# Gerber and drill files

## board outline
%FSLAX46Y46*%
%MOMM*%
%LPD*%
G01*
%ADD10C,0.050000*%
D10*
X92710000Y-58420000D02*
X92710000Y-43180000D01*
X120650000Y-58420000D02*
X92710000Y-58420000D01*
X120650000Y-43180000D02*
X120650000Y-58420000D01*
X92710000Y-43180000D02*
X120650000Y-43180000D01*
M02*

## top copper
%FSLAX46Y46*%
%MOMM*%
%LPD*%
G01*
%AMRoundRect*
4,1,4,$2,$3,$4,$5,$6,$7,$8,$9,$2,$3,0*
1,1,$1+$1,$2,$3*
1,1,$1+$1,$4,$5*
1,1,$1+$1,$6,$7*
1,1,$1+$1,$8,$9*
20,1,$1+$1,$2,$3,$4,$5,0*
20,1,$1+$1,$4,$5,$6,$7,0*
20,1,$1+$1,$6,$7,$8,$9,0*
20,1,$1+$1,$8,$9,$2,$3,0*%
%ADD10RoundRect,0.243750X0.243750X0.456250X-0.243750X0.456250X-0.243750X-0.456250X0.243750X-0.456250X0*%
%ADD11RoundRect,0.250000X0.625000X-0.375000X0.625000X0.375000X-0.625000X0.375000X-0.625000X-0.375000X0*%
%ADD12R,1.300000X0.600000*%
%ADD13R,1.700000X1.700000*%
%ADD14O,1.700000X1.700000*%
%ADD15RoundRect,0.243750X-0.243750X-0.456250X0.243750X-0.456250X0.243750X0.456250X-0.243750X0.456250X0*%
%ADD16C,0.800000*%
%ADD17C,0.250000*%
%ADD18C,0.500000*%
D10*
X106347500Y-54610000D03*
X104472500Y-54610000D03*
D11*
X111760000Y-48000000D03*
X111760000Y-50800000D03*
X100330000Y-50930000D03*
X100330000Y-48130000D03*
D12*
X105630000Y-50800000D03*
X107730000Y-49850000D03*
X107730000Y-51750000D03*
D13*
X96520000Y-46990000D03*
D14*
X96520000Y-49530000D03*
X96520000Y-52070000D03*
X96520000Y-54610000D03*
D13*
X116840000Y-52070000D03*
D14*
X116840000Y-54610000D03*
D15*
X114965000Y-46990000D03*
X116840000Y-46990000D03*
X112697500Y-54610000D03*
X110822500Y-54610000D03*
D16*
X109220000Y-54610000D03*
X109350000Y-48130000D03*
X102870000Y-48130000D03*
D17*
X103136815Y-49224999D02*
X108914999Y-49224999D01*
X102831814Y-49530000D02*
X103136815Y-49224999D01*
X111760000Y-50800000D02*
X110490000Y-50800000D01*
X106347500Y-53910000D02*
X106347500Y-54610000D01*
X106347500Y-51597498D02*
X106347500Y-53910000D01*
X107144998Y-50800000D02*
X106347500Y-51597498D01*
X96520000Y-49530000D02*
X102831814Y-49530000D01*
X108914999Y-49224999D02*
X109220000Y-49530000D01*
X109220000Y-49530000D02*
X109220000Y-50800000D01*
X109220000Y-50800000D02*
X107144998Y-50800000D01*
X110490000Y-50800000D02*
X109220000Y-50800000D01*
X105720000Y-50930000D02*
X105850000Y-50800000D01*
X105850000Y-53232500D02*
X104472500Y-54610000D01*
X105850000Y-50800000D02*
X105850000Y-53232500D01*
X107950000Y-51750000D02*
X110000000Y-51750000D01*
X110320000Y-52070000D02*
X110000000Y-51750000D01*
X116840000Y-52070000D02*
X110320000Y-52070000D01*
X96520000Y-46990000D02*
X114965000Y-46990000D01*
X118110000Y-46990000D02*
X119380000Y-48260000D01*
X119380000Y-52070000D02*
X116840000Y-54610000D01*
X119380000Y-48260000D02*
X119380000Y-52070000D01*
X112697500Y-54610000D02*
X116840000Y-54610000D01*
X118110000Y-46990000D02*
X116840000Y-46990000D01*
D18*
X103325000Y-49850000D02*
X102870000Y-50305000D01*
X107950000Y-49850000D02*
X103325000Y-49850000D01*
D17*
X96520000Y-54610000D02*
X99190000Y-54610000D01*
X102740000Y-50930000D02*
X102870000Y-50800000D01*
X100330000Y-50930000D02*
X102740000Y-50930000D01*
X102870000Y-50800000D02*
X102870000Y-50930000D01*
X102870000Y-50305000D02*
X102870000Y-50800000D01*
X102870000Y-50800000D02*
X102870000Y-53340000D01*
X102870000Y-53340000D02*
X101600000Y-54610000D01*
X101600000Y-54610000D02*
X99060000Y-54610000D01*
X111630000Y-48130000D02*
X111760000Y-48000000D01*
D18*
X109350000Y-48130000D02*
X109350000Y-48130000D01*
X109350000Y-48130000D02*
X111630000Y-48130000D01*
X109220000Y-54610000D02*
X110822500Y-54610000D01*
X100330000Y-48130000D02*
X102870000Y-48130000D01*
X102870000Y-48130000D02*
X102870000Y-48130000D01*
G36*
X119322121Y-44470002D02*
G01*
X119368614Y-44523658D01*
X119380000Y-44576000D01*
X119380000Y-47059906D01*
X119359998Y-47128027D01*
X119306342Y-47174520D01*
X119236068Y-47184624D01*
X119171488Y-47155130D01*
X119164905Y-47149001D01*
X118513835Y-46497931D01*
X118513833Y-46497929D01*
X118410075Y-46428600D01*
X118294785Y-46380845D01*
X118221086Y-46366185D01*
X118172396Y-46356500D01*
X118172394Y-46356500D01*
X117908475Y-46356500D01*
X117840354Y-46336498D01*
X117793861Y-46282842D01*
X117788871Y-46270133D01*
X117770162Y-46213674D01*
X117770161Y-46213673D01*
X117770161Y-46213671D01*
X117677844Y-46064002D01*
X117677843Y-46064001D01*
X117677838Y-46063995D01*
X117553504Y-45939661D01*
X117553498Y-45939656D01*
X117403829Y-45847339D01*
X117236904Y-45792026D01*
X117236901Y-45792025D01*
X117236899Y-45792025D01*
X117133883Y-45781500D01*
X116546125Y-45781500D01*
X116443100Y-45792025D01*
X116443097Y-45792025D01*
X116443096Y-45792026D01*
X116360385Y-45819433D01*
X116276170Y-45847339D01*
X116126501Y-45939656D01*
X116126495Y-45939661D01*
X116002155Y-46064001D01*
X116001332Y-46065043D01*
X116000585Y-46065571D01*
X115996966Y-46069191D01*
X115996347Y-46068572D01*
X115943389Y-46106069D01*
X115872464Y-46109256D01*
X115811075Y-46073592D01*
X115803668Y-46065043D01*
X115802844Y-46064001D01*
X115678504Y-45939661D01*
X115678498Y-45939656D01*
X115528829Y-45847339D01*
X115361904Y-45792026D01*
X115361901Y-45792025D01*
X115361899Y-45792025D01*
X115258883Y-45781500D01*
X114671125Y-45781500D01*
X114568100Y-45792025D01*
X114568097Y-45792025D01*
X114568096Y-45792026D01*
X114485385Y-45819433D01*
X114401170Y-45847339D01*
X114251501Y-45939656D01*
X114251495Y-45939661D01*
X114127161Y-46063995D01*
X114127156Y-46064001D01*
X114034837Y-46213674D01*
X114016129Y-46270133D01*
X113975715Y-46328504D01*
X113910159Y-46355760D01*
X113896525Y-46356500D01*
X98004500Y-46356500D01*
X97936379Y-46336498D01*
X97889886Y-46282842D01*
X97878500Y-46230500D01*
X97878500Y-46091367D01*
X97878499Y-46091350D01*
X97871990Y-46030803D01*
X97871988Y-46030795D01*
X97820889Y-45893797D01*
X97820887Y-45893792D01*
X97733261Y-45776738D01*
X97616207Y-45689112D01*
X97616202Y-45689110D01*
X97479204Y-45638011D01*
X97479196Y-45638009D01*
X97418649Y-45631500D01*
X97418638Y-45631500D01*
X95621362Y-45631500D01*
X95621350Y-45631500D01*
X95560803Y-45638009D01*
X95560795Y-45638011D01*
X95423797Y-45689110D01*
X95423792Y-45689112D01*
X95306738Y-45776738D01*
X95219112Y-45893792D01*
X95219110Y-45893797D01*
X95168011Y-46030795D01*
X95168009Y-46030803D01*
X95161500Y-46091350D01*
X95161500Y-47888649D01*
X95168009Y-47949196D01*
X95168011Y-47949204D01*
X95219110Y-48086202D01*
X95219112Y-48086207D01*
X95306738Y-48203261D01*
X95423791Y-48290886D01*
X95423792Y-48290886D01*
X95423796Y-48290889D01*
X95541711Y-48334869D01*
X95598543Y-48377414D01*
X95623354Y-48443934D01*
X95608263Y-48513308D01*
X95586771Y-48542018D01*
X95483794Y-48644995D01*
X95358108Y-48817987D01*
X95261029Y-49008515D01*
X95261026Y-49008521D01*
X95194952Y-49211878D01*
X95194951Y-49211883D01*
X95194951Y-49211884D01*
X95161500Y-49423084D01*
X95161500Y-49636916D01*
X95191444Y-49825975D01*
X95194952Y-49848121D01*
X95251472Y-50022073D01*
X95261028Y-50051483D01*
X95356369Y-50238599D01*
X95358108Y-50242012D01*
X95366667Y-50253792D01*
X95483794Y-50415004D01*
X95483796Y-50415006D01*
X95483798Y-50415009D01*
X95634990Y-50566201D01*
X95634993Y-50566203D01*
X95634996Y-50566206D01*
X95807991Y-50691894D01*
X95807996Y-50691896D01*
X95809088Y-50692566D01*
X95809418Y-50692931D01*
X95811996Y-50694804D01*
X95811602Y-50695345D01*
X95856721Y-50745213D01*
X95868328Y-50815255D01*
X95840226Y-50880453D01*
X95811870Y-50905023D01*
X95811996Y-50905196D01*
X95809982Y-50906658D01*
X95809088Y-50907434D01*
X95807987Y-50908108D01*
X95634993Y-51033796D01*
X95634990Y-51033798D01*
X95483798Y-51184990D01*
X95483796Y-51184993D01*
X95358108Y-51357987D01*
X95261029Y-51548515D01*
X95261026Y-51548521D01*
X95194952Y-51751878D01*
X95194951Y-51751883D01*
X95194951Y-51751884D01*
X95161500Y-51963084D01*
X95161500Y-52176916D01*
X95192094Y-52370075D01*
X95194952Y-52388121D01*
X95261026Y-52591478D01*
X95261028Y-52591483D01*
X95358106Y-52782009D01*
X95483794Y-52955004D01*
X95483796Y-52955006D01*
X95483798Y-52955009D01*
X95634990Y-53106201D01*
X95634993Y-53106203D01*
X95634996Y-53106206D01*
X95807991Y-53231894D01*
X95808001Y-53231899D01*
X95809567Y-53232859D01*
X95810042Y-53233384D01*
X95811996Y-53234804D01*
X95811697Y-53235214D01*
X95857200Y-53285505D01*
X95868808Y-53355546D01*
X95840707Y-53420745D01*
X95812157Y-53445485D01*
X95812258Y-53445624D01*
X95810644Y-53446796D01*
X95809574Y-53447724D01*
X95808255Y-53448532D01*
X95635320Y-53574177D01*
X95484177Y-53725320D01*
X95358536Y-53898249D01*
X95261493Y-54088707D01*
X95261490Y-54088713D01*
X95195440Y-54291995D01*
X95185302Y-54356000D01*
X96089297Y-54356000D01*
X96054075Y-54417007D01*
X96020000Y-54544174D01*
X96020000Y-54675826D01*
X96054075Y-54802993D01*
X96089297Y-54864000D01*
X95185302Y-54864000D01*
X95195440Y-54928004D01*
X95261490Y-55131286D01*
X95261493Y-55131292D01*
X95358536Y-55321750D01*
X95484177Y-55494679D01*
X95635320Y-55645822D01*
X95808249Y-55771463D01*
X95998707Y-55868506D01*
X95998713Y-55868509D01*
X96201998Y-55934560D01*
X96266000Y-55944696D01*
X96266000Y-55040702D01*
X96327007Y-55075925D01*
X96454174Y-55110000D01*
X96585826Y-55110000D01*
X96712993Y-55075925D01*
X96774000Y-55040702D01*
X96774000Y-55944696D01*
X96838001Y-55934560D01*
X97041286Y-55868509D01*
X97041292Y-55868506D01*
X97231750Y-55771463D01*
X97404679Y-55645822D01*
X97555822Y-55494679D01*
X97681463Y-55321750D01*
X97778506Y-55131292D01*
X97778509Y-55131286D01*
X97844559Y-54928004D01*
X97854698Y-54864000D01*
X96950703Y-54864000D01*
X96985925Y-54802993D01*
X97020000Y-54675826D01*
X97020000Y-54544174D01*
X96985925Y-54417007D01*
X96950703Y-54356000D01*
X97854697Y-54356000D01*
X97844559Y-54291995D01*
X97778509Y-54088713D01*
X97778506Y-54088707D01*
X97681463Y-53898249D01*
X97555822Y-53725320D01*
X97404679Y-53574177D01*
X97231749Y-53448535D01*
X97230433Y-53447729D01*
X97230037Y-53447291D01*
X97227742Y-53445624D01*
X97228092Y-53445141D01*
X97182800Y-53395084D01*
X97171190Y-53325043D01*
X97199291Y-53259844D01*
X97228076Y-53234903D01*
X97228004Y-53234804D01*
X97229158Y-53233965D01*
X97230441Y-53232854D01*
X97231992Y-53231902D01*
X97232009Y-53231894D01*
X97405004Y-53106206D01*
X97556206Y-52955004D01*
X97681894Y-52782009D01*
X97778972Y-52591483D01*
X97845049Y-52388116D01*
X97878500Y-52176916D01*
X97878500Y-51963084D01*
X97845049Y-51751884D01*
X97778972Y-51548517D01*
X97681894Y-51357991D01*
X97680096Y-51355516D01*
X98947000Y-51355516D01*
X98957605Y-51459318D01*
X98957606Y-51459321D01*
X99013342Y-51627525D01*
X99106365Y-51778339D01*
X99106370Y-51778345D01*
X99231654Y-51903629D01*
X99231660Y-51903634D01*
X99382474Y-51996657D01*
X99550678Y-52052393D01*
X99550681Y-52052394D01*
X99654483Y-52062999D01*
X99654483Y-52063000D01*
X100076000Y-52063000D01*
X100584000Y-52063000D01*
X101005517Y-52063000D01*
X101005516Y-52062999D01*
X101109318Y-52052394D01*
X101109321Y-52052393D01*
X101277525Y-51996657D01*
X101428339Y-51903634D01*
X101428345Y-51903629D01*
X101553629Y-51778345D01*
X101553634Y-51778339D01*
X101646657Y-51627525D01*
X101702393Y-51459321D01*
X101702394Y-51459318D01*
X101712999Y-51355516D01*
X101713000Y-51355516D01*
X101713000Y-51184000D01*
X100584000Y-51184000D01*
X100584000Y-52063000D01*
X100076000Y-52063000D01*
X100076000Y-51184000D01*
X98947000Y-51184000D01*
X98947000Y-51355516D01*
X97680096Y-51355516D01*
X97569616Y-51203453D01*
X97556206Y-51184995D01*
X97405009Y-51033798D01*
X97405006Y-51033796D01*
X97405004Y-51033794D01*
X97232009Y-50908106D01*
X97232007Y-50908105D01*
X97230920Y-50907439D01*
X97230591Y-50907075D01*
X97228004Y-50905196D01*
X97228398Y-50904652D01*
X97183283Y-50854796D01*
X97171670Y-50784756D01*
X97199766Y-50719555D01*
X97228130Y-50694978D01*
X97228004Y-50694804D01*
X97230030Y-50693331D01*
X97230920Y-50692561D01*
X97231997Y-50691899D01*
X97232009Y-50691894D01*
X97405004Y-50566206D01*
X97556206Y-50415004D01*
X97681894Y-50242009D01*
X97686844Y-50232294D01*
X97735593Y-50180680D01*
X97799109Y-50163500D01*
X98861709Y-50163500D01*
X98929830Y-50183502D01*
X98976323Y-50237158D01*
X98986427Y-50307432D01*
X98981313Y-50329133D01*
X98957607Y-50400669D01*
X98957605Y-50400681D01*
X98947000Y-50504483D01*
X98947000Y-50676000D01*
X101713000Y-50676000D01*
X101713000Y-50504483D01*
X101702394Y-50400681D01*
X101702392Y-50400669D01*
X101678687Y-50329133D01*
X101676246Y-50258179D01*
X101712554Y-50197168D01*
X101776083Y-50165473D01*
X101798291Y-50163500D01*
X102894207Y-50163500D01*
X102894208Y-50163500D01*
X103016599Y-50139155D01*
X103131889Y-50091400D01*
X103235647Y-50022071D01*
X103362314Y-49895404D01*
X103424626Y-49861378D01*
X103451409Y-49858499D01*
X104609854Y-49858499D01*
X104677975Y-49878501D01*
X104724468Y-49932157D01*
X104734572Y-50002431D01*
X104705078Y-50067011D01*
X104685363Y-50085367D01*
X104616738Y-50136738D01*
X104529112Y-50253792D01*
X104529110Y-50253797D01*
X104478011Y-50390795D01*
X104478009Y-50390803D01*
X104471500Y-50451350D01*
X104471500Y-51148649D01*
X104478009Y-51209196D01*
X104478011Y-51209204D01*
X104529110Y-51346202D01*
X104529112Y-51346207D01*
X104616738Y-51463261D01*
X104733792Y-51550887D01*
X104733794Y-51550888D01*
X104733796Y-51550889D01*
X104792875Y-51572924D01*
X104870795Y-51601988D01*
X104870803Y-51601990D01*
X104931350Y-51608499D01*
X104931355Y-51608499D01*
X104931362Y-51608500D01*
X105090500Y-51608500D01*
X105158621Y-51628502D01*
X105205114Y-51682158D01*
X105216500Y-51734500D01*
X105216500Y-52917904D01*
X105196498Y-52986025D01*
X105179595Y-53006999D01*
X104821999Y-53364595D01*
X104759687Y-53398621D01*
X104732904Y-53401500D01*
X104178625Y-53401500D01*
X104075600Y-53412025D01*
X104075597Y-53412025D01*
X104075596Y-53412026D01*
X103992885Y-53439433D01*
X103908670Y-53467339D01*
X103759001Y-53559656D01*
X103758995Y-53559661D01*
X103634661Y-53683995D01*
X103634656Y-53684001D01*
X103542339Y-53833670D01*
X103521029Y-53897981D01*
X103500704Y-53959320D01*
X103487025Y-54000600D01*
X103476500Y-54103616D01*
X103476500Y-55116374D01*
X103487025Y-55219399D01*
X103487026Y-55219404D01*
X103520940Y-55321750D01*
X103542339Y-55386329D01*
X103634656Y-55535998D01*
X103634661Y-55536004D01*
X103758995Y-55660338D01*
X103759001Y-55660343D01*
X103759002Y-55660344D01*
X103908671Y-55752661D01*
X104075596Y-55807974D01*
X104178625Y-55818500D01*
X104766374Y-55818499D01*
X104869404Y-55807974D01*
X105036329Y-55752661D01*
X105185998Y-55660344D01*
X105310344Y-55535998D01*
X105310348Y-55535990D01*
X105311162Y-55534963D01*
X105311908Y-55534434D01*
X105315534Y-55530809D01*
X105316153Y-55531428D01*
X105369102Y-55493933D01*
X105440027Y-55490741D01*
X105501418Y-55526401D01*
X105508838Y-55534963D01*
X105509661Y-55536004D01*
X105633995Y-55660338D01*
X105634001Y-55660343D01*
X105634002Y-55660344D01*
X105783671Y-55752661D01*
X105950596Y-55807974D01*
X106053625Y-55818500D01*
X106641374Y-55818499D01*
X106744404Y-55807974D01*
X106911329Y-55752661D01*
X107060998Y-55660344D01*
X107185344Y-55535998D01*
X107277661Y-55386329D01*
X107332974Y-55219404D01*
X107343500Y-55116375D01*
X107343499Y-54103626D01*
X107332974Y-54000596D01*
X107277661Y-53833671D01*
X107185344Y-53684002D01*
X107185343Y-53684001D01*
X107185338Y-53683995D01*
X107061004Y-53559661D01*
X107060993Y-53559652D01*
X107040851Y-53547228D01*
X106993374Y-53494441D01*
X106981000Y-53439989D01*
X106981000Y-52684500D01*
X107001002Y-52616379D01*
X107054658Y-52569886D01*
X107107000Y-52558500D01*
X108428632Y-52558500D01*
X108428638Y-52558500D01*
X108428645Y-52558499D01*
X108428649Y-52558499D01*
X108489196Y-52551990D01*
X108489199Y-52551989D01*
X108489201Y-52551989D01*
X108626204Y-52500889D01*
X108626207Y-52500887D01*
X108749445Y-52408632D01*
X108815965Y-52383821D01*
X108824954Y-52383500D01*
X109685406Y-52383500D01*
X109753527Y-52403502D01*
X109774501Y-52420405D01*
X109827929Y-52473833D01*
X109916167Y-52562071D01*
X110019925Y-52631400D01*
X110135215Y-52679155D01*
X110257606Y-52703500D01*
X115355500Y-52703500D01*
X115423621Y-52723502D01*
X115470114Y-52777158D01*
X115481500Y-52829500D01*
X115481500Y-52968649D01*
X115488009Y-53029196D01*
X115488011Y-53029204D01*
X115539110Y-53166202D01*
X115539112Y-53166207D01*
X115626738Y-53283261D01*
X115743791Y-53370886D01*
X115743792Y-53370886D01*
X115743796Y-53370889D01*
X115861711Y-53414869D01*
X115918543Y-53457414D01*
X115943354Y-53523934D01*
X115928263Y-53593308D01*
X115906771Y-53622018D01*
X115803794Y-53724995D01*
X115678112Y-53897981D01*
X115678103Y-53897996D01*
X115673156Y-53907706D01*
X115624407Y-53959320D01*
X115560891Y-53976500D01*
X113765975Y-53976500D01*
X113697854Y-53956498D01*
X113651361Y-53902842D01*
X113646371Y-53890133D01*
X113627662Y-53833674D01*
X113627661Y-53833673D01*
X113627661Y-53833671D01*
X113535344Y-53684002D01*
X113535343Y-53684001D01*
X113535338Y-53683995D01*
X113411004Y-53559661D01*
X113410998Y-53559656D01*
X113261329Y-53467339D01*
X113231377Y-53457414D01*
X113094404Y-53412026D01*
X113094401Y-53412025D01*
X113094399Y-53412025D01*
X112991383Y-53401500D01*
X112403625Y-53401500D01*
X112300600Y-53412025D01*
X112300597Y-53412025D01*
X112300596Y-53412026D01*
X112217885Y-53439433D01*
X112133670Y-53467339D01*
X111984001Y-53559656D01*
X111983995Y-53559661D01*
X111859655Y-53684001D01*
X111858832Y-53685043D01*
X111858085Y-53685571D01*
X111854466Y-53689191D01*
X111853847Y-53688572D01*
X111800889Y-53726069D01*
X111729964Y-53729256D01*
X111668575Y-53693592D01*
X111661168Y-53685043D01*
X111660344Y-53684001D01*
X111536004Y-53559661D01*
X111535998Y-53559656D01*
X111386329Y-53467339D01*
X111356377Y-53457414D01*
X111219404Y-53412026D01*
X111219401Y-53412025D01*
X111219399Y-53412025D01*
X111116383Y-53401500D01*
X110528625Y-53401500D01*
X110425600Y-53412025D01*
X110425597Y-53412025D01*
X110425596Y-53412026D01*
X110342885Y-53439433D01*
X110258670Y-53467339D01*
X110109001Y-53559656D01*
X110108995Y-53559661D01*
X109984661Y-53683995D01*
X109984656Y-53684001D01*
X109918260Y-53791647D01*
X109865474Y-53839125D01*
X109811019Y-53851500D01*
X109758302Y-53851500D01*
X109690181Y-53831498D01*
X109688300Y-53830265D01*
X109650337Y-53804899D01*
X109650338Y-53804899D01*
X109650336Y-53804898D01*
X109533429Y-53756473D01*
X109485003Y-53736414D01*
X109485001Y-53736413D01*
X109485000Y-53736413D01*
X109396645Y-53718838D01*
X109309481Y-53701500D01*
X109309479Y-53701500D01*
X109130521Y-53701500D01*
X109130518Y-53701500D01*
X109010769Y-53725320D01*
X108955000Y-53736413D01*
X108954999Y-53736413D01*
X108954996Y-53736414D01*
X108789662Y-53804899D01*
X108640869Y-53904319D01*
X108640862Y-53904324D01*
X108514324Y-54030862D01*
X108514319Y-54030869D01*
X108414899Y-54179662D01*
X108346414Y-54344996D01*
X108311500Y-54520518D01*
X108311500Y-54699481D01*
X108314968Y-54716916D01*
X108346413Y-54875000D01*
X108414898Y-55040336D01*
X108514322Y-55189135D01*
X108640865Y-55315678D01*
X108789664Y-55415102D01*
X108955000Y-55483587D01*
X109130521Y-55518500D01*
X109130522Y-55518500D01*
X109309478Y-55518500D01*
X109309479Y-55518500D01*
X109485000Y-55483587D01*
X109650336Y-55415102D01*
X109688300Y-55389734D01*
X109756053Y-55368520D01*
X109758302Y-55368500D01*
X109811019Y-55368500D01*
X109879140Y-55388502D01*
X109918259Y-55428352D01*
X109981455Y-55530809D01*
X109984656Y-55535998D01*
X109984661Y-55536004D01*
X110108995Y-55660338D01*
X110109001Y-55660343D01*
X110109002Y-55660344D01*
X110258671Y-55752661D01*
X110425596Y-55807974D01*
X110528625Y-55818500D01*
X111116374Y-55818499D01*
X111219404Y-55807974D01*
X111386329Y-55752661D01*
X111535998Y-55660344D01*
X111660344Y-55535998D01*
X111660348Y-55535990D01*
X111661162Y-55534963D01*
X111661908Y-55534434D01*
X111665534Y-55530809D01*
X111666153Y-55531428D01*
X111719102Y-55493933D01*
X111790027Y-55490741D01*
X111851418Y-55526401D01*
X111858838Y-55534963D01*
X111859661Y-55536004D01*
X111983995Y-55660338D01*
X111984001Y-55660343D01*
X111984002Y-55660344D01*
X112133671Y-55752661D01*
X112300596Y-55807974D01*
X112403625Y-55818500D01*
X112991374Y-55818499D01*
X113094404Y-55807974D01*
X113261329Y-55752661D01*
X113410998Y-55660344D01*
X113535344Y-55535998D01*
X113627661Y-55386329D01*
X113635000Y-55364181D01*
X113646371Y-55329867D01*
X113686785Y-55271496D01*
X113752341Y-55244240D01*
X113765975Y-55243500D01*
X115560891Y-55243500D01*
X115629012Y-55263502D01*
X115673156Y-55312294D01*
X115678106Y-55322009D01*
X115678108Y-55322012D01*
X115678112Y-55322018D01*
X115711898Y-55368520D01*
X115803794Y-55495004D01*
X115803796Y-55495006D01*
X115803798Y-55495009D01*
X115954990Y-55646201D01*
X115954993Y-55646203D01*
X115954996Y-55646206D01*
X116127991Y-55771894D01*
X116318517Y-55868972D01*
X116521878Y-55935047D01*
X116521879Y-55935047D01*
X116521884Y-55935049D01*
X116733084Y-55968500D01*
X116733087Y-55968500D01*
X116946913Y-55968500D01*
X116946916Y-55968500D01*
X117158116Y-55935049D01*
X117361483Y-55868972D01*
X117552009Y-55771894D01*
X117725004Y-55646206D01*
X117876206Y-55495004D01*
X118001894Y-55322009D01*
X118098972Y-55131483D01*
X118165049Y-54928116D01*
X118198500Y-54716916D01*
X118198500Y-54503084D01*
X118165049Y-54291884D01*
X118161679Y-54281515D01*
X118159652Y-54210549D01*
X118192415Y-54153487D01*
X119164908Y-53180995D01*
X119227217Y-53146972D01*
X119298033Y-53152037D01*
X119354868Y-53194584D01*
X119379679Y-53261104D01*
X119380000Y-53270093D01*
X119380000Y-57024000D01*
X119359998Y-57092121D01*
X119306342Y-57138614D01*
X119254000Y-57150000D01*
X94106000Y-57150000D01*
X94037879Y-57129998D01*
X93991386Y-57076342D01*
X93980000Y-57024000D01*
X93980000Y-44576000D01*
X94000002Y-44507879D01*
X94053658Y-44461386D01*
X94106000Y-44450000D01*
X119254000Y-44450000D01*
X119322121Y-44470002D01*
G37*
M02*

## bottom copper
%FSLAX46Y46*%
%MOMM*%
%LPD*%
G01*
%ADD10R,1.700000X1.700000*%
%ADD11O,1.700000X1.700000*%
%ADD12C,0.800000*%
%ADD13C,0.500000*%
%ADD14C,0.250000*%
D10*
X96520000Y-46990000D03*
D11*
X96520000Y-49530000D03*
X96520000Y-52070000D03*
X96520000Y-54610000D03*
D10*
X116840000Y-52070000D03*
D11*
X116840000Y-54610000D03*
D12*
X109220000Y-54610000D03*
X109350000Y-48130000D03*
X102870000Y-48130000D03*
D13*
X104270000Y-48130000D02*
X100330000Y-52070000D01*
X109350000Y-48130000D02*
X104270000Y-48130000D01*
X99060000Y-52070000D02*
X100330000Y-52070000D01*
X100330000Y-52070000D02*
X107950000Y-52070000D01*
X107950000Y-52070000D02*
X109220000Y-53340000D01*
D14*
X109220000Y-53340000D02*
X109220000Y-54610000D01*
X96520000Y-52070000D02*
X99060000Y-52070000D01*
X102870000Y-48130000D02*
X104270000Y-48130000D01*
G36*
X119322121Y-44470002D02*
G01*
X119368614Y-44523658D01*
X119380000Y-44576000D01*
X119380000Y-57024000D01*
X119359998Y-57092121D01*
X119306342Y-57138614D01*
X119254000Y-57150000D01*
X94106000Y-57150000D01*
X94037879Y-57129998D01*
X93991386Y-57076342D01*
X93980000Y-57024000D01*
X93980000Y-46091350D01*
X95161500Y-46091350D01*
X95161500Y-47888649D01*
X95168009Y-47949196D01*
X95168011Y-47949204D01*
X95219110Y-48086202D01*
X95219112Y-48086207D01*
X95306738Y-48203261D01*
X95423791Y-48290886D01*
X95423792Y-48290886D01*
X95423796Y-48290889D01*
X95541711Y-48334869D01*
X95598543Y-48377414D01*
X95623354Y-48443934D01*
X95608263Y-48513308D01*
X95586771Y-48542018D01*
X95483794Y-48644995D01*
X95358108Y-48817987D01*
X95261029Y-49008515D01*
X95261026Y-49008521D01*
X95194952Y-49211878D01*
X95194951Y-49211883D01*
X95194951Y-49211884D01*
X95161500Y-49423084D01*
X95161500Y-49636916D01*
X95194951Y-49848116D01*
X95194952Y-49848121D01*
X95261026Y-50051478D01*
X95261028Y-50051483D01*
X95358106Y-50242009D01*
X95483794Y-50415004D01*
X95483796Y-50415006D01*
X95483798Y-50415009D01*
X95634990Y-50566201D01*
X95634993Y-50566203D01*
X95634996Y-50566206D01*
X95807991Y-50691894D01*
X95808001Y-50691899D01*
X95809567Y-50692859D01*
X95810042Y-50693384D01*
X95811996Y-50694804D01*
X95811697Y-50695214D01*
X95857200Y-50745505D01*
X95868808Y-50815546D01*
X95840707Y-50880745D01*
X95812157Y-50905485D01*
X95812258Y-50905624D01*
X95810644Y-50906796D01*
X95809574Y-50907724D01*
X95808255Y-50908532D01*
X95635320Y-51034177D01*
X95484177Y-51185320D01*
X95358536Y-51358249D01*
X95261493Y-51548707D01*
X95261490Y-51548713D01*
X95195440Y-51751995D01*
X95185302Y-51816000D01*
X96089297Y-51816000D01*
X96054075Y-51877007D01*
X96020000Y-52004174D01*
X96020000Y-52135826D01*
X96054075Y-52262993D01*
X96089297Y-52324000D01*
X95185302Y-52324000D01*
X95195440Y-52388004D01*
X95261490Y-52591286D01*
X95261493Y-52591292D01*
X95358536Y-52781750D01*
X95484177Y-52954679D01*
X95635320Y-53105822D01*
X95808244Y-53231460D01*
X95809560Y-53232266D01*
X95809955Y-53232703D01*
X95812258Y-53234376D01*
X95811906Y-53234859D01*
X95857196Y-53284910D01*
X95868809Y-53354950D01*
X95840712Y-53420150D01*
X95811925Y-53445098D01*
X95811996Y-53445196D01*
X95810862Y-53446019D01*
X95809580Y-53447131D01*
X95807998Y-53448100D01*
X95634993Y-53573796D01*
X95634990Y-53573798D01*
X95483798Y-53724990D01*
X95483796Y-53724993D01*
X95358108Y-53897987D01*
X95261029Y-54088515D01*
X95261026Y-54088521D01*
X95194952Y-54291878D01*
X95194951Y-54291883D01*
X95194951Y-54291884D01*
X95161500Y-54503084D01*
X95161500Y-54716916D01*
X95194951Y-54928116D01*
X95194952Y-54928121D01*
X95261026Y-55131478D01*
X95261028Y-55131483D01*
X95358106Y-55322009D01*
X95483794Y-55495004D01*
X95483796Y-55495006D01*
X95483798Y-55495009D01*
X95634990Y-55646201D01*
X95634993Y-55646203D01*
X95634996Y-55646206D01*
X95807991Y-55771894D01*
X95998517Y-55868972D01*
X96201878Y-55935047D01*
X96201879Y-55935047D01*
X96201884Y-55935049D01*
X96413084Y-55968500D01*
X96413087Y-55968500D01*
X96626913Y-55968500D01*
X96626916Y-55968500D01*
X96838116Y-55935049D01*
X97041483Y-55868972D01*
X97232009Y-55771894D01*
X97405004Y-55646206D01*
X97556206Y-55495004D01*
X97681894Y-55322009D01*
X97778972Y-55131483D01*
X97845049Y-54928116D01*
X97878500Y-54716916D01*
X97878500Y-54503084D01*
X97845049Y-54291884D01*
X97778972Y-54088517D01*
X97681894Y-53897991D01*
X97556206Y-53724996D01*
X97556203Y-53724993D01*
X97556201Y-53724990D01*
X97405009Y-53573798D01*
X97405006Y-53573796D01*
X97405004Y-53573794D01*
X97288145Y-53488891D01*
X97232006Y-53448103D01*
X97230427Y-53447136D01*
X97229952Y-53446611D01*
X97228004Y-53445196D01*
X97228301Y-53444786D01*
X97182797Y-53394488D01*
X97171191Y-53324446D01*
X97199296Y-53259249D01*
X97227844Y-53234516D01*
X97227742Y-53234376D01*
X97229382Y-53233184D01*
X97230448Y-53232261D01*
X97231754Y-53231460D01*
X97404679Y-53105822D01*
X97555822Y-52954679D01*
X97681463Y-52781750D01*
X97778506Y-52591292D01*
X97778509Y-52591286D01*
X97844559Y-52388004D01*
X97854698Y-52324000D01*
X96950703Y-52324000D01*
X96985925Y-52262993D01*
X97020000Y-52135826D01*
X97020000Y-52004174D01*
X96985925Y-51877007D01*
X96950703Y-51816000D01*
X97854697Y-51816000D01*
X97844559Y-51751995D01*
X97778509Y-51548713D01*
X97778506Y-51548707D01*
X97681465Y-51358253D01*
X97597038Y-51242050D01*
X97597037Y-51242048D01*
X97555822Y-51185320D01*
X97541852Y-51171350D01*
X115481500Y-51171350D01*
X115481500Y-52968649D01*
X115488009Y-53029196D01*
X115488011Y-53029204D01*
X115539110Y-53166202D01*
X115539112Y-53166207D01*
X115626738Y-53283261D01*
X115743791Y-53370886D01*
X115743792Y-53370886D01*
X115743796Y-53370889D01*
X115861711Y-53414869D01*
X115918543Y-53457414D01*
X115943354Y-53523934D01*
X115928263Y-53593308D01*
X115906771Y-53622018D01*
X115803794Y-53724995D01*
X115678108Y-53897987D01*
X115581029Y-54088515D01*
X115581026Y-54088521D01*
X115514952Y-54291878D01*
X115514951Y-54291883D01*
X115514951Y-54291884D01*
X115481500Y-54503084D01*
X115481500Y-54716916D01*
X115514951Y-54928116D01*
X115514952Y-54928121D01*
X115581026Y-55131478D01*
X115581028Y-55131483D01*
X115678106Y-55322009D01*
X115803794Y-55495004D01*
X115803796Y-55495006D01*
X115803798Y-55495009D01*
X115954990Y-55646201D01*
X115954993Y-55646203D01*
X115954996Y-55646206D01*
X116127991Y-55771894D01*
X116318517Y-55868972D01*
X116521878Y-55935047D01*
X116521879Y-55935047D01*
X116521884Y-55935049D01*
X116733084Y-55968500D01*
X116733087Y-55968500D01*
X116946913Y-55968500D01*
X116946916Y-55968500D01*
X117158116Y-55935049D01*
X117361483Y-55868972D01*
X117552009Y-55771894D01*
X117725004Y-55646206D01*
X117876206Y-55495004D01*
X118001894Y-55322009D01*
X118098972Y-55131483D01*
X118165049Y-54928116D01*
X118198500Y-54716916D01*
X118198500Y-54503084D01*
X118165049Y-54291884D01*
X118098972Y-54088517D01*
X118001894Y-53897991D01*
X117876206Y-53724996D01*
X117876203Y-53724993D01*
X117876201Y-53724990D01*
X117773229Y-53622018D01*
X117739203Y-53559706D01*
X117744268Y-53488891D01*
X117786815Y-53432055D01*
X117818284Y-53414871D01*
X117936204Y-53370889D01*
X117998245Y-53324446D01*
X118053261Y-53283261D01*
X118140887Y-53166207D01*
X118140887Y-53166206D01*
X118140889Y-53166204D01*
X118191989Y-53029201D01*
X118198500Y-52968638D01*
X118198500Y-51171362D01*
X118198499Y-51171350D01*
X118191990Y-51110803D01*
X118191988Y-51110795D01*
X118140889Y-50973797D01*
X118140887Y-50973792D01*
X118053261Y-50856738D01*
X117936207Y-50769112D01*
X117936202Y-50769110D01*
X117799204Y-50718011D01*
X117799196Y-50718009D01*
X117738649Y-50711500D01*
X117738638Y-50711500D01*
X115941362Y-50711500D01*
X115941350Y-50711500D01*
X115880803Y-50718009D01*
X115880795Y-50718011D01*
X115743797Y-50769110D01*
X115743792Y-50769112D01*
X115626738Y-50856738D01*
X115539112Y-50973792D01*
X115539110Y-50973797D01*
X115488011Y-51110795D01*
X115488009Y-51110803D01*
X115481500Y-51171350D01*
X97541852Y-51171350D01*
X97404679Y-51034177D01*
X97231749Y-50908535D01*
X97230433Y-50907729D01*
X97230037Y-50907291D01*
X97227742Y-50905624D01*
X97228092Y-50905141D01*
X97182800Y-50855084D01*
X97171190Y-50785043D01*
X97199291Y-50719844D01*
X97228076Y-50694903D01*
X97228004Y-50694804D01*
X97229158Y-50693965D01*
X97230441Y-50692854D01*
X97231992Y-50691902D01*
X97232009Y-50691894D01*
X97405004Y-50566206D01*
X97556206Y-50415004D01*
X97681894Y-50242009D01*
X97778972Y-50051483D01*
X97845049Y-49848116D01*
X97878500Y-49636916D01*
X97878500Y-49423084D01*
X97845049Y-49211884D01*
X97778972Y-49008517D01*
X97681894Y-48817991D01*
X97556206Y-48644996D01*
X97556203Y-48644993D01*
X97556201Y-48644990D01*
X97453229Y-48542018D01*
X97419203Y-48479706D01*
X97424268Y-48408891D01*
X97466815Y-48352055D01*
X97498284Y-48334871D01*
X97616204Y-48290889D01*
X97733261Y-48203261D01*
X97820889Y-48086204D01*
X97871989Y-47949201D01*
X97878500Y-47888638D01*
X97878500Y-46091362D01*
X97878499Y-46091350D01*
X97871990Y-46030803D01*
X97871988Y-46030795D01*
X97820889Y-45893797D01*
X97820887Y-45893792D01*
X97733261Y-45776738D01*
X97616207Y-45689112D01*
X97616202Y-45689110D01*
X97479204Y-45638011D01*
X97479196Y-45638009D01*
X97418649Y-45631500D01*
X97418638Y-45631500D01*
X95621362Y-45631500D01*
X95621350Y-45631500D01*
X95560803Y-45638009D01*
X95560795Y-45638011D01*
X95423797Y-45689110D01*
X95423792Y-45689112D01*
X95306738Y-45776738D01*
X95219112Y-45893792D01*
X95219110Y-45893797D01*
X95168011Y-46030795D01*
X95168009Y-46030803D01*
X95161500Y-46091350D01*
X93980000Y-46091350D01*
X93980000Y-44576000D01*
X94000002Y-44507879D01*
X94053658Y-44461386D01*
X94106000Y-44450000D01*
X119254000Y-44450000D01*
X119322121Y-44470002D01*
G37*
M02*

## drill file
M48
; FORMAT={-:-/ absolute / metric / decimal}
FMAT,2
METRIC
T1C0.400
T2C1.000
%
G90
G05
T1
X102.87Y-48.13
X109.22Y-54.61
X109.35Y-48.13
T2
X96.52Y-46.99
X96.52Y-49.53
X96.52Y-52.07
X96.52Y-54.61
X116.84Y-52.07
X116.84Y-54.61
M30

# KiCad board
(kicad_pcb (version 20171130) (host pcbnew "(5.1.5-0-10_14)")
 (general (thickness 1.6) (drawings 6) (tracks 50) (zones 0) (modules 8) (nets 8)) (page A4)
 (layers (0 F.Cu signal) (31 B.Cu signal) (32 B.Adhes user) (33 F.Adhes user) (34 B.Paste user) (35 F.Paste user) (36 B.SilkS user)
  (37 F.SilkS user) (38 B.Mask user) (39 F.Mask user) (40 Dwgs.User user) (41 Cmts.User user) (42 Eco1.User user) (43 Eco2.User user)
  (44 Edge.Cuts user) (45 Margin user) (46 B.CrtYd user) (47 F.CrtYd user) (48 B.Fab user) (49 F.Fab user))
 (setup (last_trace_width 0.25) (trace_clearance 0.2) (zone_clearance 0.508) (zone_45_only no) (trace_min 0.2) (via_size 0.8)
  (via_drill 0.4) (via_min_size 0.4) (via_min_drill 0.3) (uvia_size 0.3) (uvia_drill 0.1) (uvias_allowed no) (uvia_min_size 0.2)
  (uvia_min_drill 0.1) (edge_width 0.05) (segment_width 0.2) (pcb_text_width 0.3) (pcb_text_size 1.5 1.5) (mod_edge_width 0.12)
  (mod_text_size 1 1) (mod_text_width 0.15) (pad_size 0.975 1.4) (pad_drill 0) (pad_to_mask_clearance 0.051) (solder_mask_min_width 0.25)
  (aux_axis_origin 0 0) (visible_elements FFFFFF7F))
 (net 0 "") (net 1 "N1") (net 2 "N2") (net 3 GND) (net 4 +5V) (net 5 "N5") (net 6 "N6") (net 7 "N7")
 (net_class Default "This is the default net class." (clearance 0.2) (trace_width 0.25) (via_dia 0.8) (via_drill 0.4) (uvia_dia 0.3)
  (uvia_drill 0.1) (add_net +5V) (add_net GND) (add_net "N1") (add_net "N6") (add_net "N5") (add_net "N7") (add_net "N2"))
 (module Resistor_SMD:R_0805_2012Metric (layer F.Cu) (at 105.41 54.61 180)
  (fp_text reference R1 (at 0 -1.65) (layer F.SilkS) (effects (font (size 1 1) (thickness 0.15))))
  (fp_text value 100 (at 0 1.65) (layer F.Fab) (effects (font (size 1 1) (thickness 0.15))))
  (pad 1 smd roundrect (at -0.9375 0 180) (size 0.975 1.4) (layers F.Cu F.Paste F.Mask) (roundrect_rratio 0.25) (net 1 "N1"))
  (pad 2 smd roundrect (at 0.9375 0 180) (size 0.975 1.4) (layers F.Cu F.Paste F.Mask) (roundrect_rratio 0.25) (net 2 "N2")))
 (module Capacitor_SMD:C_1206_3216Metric (layer F.Cu) (at 111.76 49.4 90)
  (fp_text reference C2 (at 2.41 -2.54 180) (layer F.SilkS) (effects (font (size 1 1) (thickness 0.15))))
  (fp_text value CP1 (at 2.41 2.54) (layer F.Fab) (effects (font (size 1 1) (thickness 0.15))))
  (pad 2 smd roundrect (at 1.4 0 90) (size 1.25 1.75) (layers F.Cu F.Paste F.Mask) (roundrect_rratio 0.2) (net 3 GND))
  (pad 1 smd roundrect (at -1.4 0 90) (size 1.25 1.75) (layers F.Cu F.Paste F.Mask) (roundrect_rratio 0.2) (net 1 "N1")))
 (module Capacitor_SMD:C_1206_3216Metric (layer F.Cu) (at 100.33 49.53 90)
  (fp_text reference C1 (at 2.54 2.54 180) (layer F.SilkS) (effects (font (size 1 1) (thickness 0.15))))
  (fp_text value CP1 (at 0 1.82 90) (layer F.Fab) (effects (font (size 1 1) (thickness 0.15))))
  (pad 1 smd roundrect (at -1.4 0 90) (size 1.25 1.75) (layers F.Cu F.Paste F.Mask) (roundrect_rratio 0.2) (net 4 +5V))
  (pad 2 smd roundrect (at 1.4 0 90) (size 1.25 1.75) (layers F.Cu F.Paste F.Mask) (roundrect_rratio 0.2) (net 3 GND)))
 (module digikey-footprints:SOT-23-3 (layer F.Cu) (at 106.68 50.8 180)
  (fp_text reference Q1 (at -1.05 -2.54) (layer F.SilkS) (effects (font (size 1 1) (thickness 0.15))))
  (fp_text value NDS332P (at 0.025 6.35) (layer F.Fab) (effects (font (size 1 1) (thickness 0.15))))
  (pad 3 smd rect (at 1.05 0 180) (size 1.3 0.6) (layers F.Cu F.Paste F.Mask) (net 2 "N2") (solder_mask_margin 0.07))
  (pad 2 smd rect (at -1.05 0.95 180) (size 1.3 0.6) (layers F.Cu F.Paste F.Mask) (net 4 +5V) (solder_mask_margin 0.07))
  (pad 1 smd rect (at -1.05 -0.95 180) (size 1.3 0.6) (layers F.Cu F.Paste F.Mask) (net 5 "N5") (solder_mask_margin 0.07)))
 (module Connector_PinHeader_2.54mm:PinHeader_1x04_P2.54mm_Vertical (layer F.Cu) (at 96.52 46.99)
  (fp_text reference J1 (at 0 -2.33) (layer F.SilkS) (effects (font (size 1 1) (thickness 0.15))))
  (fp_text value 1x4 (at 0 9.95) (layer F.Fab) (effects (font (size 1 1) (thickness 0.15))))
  (pad 1 thru_hole rect (at 0 0) (size 1.7 1.7) (drill 1) (layers *.Cu *.Mask) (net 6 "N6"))
  (pad 2 thru_hole oval (at 0 2.54) (size 1.7 1.7) (drill 1) (layers *.Cu *.Mask) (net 1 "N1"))
  (pad 3 thru_hole oval (at 0 5.08) (size 1.7 1.7) (drill 1) (layers *.Cu *.Mask) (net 3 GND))
  (pad 4 thru_hole oval (at 0 7.62) (size 1.7 1.7) (drill 1) (layers *.Cu *.Mask) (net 4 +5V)))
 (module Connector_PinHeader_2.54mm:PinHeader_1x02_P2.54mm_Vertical (layer F.Cu) (at 116.84 52.07)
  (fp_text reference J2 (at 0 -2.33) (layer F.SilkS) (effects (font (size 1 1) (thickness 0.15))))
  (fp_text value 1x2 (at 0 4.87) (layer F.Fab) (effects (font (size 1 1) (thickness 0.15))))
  (pad 1 thru_hole rect (at 0 0) (size 1.7 1.7) (drill 1) (layers *.Cu *.Mask) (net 5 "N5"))
  (pad 2 thru_hole oval (at 0 2.54) (size 1.7 1.7) (drill 1) (layers *.Cu *.Mask) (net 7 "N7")))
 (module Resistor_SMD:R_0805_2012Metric (layer F.Cu) (at 115.9025 46.99)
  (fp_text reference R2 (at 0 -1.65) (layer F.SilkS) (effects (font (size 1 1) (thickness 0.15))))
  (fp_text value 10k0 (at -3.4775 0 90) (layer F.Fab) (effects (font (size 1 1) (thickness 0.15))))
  (pad 1 smd roundrect (at -0.9375 0) (size 0.975 1.4) (layers F.Cu F.Paste F.Mask) (roundrect_rratio 0.25) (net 6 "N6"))
  (pad 2 smd roundrect (at 0.9375 0) (size 0.975 1.4) (layers F.Cu F.Paste F.Mask) (roundrect_rratio 0.25) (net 7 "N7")))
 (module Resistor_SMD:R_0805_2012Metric (layer F.Cu) (at 111.76 54.61)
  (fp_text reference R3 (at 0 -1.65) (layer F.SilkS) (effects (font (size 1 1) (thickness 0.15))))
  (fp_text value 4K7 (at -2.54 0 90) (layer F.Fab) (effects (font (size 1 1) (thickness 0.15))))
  (pad 2 smd roundrect (at 0.9375 0) (size 0.975 1.4) (layers F.Cu F.Paste F.Mask) (roundrect_rratio 0.25) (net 7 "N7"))
  (pad 1 smd roundrect (at -0.9375 0) (size 0.975 1.4) (layers F.Cu F.Paste F.Mask) (roundrect_rratio 0.25) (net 3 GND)))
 (gr_line (start 92.71 58.42) (end 92.71 43.18) (layer Edge.Cuts) (width 0.05))
 (gr_line (start 120.65 58.42) (end 92.71 58.42) (layer Edge.Cuts) (width 0.05))
 (gr_line (start 120.65 43.18) (end 120.65 58.42) (layer Edge.Cuts) (width 0.05))
 (gr_line (start 92.71 43.18) (end 120.65 43.18) (layer Edge.Cuts) (width 0.05))
 (segment (start 103.136815 49.224999) (end 108.914999 49.224999) (width 0.25) (layer F.Cu) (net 1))
 (segment (start 102.831814 49.53) (end 103.136815 49.224999) (width 0.25) (layer F.Cu) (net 1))
 (segment (start 111.76 50.8) (end 110.49 50.8) (width 0.25) (layer F.Cu) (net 1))
 (segment (start 106.3475 53.91) (end 106.3475 54.61) (width 0.25) (layer F.Cu) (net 1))
 (segment (start 106.3475 51.597498) (end 106.3475 53.91) (width 0.25) (layer F.Cu) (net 1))
 (segment (start 107.144998 50.8) (end 106.3475 51.597498) (width 0.25) (layer F.Cu) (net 1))
 (segment (start 96.52 49.53) (end 102.831814 49.53) (width 0.25) (layer F.Cu) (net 1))
 (segment (start 108.914999 49.224999) (end 109.22 49.53) (width 0.25) (layer F.Cu) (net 1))
 (segment (start 109.22 49.53) (end 109.22 50.8) (width 0.25) (layer F.Cu) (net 1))
 (segment (start 109.22 50.8) (end 107.144998 50.8) (width 0.25) (layer F.Cu) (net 1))
 (segment (start 110.49 50.8) (end 109.22 50.8) (width 0.25) (layer F.Cu) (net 1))
 (segment (start 105.72 50.93) (end 105.85 50.8) (width 0.25) (layer F.Cu) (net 2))
 (segment (start 105.85 53.2325) (end 104.4725 54.61) (width 0.25) (layer F.Cu) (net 2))
 (segment (start 105.85 50.8) (end 105.85 53.2325) (width 0.25) (layer F.Cu) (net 2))
 (segment (start 107.95 51.75) (end 110 51.75) (width 0.25) (layer F.Cu) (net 5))
 (segment (start 110.32 52.07) (end 110 51.75) (width 0.25) (layer F.Cu) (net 5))
 (segment (start 116.84 52.07) (end 110.32 52.07) (width 0.25) (layer F.Cu) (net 5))
 (segment (start 96.52 46.99) (end 114.965 46.99) (width 0.25) (layer F.Cu) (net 6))
 (segment (start 118.11 46.99) (end 119.38 48.26) (width 0.25) (layer F.Cu) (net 7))
 (segment (start 119.38 52.07) (end 116.84 54.61) (width 0.25) (layer F.Cu) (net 7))
 (segment (start 119.38 48.26) (end 119.38 52.07) (width 0.25) (layer F.Cu) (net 7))
 (segment (start 112.6975 54.61) (end 116.84 54.61) (width 0.25) (layer F.Cu) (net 7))
 (segment (start 118.11 46.99) (end 116.84 46.99) (width 0.25) (layer F.Cu) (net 7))
 (segment (start 103.325 49.85) (end 102.87 50.305) (width 0.5) (layer F.Cu) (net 4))
 (segment (start 107.95 49.85) (end 103.325 49.85) (width 0.5) (layer F.Cu) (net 4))
 (segment (start 96.52 54.61) (end 99.19 54.61) (width 0.25) (layer F.Cu) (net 4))
 (segment (start 102.74 50.93) (end 102.87 50.8) (width 0.25) (layer F.Cu) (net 4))
 (segment (start 100.33 50.93) (end 102.74 50.93) (width 0.25) (layer F.Cu) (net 4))
 (segment (start 102.87 50.8) (end 102.87 50.93) (width 0.25) (layer F.Cu) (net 4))
 (segment (start 102.87 50.305) (end 102.87 50.8) (width 0.25) (layer F.Cu) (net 4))
 (segment (start 102.87 50.8) (end 102.87 53.34) (width 0.25) (layer F.Cu) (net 4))
 (segment (start 102.87 53.34) (end 101.6 54.61) (width 0.25) (layer F.Cu) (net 4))
 (segment (start 101.6 54.61) (end 99.06 54.61) (width 0.25) (layer F.Cu) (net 4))
 (segment (start 111.63 48.13) (end 111.76 48) (width 0.25) (layer F.Cu) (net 3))
 (segment (start 109.35 48.13) (end 109.35 48.13) (width 0.5) (layer F.Cu) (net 3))
 (segment (start 104.27 48.13) (end 100.33 52.07) (width 0.5) (layer B.Cu) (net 3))
 (segment (start 109.35 48.13) (end 104.27 48.13) (width 0.5) (layer B.Cu) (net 3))
 (segment (start 99.06 52.07) (end 100.33 52.07) (width 0.5) (layer B.Cu) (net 3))
 (via (at 109.22 54.61) (size 0.8) (drill 0.4) (layers F.Cu B.Cu) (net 3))
 (segment (start 109.35 48.13) (end 111.63 48.13) (width 0.5) (layer F.Cu) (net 3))
 (via (at 109.35 48.13) (size 0.8) (drill 0.4) (layers F.Cu B.Cu) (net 3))
 (segment (start 100.33 52.07) (end 107.95 52.07) (width 0.5) (layer B.Cu) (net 3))
 (segment (start 107.95 52.07) (end 109.22 53.34) (width 0.5) (layer B.Cu) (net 3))
 (segment (start 109.22 54.61) (end 110.8225 54.61) (width 0.5) (layer F.Cu) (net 3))
 (segment (start 100.33 48.13) (end 102.87 48.13) (width 0.5) (layer F.Cu) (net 3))
 (segment (start 102.87 48.13) (end 102.87 48.13) (width 0.5) (layer F.Cu) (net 3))
 (via (at 102.87 48.13) (size 0.8) (drill 0.4) (layers F.Cu B.Cu) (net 3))
 (segment (start 109.22 53.34) (end 109.22 54.61) (width 0.25) (layer B.Cu) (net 3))
 (segment (start 96.52 52.07) (end 99.06 52.07) (width 0.25) (layer B.Cu) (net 3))
 (segment (start 102.87 48.13) (end 104.27 48.13) (width 0.25) (layer B.Cu) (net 3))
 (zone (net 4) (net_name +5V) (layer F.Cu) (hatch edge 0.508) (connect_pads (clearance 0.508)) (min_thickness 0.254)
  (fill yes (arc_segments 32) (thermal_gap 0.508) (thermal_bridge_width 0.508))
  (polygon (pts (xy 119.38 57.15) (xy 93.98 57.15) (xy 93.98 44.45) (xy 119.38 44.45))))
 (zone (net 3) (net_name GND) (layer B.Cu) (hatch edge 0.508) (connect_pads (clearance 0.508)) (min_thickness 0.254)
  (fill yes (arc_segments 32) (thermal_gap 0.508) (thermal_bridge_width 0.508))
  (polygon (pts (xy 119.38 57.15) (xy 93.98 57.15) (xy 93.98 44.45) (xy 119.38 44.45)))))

